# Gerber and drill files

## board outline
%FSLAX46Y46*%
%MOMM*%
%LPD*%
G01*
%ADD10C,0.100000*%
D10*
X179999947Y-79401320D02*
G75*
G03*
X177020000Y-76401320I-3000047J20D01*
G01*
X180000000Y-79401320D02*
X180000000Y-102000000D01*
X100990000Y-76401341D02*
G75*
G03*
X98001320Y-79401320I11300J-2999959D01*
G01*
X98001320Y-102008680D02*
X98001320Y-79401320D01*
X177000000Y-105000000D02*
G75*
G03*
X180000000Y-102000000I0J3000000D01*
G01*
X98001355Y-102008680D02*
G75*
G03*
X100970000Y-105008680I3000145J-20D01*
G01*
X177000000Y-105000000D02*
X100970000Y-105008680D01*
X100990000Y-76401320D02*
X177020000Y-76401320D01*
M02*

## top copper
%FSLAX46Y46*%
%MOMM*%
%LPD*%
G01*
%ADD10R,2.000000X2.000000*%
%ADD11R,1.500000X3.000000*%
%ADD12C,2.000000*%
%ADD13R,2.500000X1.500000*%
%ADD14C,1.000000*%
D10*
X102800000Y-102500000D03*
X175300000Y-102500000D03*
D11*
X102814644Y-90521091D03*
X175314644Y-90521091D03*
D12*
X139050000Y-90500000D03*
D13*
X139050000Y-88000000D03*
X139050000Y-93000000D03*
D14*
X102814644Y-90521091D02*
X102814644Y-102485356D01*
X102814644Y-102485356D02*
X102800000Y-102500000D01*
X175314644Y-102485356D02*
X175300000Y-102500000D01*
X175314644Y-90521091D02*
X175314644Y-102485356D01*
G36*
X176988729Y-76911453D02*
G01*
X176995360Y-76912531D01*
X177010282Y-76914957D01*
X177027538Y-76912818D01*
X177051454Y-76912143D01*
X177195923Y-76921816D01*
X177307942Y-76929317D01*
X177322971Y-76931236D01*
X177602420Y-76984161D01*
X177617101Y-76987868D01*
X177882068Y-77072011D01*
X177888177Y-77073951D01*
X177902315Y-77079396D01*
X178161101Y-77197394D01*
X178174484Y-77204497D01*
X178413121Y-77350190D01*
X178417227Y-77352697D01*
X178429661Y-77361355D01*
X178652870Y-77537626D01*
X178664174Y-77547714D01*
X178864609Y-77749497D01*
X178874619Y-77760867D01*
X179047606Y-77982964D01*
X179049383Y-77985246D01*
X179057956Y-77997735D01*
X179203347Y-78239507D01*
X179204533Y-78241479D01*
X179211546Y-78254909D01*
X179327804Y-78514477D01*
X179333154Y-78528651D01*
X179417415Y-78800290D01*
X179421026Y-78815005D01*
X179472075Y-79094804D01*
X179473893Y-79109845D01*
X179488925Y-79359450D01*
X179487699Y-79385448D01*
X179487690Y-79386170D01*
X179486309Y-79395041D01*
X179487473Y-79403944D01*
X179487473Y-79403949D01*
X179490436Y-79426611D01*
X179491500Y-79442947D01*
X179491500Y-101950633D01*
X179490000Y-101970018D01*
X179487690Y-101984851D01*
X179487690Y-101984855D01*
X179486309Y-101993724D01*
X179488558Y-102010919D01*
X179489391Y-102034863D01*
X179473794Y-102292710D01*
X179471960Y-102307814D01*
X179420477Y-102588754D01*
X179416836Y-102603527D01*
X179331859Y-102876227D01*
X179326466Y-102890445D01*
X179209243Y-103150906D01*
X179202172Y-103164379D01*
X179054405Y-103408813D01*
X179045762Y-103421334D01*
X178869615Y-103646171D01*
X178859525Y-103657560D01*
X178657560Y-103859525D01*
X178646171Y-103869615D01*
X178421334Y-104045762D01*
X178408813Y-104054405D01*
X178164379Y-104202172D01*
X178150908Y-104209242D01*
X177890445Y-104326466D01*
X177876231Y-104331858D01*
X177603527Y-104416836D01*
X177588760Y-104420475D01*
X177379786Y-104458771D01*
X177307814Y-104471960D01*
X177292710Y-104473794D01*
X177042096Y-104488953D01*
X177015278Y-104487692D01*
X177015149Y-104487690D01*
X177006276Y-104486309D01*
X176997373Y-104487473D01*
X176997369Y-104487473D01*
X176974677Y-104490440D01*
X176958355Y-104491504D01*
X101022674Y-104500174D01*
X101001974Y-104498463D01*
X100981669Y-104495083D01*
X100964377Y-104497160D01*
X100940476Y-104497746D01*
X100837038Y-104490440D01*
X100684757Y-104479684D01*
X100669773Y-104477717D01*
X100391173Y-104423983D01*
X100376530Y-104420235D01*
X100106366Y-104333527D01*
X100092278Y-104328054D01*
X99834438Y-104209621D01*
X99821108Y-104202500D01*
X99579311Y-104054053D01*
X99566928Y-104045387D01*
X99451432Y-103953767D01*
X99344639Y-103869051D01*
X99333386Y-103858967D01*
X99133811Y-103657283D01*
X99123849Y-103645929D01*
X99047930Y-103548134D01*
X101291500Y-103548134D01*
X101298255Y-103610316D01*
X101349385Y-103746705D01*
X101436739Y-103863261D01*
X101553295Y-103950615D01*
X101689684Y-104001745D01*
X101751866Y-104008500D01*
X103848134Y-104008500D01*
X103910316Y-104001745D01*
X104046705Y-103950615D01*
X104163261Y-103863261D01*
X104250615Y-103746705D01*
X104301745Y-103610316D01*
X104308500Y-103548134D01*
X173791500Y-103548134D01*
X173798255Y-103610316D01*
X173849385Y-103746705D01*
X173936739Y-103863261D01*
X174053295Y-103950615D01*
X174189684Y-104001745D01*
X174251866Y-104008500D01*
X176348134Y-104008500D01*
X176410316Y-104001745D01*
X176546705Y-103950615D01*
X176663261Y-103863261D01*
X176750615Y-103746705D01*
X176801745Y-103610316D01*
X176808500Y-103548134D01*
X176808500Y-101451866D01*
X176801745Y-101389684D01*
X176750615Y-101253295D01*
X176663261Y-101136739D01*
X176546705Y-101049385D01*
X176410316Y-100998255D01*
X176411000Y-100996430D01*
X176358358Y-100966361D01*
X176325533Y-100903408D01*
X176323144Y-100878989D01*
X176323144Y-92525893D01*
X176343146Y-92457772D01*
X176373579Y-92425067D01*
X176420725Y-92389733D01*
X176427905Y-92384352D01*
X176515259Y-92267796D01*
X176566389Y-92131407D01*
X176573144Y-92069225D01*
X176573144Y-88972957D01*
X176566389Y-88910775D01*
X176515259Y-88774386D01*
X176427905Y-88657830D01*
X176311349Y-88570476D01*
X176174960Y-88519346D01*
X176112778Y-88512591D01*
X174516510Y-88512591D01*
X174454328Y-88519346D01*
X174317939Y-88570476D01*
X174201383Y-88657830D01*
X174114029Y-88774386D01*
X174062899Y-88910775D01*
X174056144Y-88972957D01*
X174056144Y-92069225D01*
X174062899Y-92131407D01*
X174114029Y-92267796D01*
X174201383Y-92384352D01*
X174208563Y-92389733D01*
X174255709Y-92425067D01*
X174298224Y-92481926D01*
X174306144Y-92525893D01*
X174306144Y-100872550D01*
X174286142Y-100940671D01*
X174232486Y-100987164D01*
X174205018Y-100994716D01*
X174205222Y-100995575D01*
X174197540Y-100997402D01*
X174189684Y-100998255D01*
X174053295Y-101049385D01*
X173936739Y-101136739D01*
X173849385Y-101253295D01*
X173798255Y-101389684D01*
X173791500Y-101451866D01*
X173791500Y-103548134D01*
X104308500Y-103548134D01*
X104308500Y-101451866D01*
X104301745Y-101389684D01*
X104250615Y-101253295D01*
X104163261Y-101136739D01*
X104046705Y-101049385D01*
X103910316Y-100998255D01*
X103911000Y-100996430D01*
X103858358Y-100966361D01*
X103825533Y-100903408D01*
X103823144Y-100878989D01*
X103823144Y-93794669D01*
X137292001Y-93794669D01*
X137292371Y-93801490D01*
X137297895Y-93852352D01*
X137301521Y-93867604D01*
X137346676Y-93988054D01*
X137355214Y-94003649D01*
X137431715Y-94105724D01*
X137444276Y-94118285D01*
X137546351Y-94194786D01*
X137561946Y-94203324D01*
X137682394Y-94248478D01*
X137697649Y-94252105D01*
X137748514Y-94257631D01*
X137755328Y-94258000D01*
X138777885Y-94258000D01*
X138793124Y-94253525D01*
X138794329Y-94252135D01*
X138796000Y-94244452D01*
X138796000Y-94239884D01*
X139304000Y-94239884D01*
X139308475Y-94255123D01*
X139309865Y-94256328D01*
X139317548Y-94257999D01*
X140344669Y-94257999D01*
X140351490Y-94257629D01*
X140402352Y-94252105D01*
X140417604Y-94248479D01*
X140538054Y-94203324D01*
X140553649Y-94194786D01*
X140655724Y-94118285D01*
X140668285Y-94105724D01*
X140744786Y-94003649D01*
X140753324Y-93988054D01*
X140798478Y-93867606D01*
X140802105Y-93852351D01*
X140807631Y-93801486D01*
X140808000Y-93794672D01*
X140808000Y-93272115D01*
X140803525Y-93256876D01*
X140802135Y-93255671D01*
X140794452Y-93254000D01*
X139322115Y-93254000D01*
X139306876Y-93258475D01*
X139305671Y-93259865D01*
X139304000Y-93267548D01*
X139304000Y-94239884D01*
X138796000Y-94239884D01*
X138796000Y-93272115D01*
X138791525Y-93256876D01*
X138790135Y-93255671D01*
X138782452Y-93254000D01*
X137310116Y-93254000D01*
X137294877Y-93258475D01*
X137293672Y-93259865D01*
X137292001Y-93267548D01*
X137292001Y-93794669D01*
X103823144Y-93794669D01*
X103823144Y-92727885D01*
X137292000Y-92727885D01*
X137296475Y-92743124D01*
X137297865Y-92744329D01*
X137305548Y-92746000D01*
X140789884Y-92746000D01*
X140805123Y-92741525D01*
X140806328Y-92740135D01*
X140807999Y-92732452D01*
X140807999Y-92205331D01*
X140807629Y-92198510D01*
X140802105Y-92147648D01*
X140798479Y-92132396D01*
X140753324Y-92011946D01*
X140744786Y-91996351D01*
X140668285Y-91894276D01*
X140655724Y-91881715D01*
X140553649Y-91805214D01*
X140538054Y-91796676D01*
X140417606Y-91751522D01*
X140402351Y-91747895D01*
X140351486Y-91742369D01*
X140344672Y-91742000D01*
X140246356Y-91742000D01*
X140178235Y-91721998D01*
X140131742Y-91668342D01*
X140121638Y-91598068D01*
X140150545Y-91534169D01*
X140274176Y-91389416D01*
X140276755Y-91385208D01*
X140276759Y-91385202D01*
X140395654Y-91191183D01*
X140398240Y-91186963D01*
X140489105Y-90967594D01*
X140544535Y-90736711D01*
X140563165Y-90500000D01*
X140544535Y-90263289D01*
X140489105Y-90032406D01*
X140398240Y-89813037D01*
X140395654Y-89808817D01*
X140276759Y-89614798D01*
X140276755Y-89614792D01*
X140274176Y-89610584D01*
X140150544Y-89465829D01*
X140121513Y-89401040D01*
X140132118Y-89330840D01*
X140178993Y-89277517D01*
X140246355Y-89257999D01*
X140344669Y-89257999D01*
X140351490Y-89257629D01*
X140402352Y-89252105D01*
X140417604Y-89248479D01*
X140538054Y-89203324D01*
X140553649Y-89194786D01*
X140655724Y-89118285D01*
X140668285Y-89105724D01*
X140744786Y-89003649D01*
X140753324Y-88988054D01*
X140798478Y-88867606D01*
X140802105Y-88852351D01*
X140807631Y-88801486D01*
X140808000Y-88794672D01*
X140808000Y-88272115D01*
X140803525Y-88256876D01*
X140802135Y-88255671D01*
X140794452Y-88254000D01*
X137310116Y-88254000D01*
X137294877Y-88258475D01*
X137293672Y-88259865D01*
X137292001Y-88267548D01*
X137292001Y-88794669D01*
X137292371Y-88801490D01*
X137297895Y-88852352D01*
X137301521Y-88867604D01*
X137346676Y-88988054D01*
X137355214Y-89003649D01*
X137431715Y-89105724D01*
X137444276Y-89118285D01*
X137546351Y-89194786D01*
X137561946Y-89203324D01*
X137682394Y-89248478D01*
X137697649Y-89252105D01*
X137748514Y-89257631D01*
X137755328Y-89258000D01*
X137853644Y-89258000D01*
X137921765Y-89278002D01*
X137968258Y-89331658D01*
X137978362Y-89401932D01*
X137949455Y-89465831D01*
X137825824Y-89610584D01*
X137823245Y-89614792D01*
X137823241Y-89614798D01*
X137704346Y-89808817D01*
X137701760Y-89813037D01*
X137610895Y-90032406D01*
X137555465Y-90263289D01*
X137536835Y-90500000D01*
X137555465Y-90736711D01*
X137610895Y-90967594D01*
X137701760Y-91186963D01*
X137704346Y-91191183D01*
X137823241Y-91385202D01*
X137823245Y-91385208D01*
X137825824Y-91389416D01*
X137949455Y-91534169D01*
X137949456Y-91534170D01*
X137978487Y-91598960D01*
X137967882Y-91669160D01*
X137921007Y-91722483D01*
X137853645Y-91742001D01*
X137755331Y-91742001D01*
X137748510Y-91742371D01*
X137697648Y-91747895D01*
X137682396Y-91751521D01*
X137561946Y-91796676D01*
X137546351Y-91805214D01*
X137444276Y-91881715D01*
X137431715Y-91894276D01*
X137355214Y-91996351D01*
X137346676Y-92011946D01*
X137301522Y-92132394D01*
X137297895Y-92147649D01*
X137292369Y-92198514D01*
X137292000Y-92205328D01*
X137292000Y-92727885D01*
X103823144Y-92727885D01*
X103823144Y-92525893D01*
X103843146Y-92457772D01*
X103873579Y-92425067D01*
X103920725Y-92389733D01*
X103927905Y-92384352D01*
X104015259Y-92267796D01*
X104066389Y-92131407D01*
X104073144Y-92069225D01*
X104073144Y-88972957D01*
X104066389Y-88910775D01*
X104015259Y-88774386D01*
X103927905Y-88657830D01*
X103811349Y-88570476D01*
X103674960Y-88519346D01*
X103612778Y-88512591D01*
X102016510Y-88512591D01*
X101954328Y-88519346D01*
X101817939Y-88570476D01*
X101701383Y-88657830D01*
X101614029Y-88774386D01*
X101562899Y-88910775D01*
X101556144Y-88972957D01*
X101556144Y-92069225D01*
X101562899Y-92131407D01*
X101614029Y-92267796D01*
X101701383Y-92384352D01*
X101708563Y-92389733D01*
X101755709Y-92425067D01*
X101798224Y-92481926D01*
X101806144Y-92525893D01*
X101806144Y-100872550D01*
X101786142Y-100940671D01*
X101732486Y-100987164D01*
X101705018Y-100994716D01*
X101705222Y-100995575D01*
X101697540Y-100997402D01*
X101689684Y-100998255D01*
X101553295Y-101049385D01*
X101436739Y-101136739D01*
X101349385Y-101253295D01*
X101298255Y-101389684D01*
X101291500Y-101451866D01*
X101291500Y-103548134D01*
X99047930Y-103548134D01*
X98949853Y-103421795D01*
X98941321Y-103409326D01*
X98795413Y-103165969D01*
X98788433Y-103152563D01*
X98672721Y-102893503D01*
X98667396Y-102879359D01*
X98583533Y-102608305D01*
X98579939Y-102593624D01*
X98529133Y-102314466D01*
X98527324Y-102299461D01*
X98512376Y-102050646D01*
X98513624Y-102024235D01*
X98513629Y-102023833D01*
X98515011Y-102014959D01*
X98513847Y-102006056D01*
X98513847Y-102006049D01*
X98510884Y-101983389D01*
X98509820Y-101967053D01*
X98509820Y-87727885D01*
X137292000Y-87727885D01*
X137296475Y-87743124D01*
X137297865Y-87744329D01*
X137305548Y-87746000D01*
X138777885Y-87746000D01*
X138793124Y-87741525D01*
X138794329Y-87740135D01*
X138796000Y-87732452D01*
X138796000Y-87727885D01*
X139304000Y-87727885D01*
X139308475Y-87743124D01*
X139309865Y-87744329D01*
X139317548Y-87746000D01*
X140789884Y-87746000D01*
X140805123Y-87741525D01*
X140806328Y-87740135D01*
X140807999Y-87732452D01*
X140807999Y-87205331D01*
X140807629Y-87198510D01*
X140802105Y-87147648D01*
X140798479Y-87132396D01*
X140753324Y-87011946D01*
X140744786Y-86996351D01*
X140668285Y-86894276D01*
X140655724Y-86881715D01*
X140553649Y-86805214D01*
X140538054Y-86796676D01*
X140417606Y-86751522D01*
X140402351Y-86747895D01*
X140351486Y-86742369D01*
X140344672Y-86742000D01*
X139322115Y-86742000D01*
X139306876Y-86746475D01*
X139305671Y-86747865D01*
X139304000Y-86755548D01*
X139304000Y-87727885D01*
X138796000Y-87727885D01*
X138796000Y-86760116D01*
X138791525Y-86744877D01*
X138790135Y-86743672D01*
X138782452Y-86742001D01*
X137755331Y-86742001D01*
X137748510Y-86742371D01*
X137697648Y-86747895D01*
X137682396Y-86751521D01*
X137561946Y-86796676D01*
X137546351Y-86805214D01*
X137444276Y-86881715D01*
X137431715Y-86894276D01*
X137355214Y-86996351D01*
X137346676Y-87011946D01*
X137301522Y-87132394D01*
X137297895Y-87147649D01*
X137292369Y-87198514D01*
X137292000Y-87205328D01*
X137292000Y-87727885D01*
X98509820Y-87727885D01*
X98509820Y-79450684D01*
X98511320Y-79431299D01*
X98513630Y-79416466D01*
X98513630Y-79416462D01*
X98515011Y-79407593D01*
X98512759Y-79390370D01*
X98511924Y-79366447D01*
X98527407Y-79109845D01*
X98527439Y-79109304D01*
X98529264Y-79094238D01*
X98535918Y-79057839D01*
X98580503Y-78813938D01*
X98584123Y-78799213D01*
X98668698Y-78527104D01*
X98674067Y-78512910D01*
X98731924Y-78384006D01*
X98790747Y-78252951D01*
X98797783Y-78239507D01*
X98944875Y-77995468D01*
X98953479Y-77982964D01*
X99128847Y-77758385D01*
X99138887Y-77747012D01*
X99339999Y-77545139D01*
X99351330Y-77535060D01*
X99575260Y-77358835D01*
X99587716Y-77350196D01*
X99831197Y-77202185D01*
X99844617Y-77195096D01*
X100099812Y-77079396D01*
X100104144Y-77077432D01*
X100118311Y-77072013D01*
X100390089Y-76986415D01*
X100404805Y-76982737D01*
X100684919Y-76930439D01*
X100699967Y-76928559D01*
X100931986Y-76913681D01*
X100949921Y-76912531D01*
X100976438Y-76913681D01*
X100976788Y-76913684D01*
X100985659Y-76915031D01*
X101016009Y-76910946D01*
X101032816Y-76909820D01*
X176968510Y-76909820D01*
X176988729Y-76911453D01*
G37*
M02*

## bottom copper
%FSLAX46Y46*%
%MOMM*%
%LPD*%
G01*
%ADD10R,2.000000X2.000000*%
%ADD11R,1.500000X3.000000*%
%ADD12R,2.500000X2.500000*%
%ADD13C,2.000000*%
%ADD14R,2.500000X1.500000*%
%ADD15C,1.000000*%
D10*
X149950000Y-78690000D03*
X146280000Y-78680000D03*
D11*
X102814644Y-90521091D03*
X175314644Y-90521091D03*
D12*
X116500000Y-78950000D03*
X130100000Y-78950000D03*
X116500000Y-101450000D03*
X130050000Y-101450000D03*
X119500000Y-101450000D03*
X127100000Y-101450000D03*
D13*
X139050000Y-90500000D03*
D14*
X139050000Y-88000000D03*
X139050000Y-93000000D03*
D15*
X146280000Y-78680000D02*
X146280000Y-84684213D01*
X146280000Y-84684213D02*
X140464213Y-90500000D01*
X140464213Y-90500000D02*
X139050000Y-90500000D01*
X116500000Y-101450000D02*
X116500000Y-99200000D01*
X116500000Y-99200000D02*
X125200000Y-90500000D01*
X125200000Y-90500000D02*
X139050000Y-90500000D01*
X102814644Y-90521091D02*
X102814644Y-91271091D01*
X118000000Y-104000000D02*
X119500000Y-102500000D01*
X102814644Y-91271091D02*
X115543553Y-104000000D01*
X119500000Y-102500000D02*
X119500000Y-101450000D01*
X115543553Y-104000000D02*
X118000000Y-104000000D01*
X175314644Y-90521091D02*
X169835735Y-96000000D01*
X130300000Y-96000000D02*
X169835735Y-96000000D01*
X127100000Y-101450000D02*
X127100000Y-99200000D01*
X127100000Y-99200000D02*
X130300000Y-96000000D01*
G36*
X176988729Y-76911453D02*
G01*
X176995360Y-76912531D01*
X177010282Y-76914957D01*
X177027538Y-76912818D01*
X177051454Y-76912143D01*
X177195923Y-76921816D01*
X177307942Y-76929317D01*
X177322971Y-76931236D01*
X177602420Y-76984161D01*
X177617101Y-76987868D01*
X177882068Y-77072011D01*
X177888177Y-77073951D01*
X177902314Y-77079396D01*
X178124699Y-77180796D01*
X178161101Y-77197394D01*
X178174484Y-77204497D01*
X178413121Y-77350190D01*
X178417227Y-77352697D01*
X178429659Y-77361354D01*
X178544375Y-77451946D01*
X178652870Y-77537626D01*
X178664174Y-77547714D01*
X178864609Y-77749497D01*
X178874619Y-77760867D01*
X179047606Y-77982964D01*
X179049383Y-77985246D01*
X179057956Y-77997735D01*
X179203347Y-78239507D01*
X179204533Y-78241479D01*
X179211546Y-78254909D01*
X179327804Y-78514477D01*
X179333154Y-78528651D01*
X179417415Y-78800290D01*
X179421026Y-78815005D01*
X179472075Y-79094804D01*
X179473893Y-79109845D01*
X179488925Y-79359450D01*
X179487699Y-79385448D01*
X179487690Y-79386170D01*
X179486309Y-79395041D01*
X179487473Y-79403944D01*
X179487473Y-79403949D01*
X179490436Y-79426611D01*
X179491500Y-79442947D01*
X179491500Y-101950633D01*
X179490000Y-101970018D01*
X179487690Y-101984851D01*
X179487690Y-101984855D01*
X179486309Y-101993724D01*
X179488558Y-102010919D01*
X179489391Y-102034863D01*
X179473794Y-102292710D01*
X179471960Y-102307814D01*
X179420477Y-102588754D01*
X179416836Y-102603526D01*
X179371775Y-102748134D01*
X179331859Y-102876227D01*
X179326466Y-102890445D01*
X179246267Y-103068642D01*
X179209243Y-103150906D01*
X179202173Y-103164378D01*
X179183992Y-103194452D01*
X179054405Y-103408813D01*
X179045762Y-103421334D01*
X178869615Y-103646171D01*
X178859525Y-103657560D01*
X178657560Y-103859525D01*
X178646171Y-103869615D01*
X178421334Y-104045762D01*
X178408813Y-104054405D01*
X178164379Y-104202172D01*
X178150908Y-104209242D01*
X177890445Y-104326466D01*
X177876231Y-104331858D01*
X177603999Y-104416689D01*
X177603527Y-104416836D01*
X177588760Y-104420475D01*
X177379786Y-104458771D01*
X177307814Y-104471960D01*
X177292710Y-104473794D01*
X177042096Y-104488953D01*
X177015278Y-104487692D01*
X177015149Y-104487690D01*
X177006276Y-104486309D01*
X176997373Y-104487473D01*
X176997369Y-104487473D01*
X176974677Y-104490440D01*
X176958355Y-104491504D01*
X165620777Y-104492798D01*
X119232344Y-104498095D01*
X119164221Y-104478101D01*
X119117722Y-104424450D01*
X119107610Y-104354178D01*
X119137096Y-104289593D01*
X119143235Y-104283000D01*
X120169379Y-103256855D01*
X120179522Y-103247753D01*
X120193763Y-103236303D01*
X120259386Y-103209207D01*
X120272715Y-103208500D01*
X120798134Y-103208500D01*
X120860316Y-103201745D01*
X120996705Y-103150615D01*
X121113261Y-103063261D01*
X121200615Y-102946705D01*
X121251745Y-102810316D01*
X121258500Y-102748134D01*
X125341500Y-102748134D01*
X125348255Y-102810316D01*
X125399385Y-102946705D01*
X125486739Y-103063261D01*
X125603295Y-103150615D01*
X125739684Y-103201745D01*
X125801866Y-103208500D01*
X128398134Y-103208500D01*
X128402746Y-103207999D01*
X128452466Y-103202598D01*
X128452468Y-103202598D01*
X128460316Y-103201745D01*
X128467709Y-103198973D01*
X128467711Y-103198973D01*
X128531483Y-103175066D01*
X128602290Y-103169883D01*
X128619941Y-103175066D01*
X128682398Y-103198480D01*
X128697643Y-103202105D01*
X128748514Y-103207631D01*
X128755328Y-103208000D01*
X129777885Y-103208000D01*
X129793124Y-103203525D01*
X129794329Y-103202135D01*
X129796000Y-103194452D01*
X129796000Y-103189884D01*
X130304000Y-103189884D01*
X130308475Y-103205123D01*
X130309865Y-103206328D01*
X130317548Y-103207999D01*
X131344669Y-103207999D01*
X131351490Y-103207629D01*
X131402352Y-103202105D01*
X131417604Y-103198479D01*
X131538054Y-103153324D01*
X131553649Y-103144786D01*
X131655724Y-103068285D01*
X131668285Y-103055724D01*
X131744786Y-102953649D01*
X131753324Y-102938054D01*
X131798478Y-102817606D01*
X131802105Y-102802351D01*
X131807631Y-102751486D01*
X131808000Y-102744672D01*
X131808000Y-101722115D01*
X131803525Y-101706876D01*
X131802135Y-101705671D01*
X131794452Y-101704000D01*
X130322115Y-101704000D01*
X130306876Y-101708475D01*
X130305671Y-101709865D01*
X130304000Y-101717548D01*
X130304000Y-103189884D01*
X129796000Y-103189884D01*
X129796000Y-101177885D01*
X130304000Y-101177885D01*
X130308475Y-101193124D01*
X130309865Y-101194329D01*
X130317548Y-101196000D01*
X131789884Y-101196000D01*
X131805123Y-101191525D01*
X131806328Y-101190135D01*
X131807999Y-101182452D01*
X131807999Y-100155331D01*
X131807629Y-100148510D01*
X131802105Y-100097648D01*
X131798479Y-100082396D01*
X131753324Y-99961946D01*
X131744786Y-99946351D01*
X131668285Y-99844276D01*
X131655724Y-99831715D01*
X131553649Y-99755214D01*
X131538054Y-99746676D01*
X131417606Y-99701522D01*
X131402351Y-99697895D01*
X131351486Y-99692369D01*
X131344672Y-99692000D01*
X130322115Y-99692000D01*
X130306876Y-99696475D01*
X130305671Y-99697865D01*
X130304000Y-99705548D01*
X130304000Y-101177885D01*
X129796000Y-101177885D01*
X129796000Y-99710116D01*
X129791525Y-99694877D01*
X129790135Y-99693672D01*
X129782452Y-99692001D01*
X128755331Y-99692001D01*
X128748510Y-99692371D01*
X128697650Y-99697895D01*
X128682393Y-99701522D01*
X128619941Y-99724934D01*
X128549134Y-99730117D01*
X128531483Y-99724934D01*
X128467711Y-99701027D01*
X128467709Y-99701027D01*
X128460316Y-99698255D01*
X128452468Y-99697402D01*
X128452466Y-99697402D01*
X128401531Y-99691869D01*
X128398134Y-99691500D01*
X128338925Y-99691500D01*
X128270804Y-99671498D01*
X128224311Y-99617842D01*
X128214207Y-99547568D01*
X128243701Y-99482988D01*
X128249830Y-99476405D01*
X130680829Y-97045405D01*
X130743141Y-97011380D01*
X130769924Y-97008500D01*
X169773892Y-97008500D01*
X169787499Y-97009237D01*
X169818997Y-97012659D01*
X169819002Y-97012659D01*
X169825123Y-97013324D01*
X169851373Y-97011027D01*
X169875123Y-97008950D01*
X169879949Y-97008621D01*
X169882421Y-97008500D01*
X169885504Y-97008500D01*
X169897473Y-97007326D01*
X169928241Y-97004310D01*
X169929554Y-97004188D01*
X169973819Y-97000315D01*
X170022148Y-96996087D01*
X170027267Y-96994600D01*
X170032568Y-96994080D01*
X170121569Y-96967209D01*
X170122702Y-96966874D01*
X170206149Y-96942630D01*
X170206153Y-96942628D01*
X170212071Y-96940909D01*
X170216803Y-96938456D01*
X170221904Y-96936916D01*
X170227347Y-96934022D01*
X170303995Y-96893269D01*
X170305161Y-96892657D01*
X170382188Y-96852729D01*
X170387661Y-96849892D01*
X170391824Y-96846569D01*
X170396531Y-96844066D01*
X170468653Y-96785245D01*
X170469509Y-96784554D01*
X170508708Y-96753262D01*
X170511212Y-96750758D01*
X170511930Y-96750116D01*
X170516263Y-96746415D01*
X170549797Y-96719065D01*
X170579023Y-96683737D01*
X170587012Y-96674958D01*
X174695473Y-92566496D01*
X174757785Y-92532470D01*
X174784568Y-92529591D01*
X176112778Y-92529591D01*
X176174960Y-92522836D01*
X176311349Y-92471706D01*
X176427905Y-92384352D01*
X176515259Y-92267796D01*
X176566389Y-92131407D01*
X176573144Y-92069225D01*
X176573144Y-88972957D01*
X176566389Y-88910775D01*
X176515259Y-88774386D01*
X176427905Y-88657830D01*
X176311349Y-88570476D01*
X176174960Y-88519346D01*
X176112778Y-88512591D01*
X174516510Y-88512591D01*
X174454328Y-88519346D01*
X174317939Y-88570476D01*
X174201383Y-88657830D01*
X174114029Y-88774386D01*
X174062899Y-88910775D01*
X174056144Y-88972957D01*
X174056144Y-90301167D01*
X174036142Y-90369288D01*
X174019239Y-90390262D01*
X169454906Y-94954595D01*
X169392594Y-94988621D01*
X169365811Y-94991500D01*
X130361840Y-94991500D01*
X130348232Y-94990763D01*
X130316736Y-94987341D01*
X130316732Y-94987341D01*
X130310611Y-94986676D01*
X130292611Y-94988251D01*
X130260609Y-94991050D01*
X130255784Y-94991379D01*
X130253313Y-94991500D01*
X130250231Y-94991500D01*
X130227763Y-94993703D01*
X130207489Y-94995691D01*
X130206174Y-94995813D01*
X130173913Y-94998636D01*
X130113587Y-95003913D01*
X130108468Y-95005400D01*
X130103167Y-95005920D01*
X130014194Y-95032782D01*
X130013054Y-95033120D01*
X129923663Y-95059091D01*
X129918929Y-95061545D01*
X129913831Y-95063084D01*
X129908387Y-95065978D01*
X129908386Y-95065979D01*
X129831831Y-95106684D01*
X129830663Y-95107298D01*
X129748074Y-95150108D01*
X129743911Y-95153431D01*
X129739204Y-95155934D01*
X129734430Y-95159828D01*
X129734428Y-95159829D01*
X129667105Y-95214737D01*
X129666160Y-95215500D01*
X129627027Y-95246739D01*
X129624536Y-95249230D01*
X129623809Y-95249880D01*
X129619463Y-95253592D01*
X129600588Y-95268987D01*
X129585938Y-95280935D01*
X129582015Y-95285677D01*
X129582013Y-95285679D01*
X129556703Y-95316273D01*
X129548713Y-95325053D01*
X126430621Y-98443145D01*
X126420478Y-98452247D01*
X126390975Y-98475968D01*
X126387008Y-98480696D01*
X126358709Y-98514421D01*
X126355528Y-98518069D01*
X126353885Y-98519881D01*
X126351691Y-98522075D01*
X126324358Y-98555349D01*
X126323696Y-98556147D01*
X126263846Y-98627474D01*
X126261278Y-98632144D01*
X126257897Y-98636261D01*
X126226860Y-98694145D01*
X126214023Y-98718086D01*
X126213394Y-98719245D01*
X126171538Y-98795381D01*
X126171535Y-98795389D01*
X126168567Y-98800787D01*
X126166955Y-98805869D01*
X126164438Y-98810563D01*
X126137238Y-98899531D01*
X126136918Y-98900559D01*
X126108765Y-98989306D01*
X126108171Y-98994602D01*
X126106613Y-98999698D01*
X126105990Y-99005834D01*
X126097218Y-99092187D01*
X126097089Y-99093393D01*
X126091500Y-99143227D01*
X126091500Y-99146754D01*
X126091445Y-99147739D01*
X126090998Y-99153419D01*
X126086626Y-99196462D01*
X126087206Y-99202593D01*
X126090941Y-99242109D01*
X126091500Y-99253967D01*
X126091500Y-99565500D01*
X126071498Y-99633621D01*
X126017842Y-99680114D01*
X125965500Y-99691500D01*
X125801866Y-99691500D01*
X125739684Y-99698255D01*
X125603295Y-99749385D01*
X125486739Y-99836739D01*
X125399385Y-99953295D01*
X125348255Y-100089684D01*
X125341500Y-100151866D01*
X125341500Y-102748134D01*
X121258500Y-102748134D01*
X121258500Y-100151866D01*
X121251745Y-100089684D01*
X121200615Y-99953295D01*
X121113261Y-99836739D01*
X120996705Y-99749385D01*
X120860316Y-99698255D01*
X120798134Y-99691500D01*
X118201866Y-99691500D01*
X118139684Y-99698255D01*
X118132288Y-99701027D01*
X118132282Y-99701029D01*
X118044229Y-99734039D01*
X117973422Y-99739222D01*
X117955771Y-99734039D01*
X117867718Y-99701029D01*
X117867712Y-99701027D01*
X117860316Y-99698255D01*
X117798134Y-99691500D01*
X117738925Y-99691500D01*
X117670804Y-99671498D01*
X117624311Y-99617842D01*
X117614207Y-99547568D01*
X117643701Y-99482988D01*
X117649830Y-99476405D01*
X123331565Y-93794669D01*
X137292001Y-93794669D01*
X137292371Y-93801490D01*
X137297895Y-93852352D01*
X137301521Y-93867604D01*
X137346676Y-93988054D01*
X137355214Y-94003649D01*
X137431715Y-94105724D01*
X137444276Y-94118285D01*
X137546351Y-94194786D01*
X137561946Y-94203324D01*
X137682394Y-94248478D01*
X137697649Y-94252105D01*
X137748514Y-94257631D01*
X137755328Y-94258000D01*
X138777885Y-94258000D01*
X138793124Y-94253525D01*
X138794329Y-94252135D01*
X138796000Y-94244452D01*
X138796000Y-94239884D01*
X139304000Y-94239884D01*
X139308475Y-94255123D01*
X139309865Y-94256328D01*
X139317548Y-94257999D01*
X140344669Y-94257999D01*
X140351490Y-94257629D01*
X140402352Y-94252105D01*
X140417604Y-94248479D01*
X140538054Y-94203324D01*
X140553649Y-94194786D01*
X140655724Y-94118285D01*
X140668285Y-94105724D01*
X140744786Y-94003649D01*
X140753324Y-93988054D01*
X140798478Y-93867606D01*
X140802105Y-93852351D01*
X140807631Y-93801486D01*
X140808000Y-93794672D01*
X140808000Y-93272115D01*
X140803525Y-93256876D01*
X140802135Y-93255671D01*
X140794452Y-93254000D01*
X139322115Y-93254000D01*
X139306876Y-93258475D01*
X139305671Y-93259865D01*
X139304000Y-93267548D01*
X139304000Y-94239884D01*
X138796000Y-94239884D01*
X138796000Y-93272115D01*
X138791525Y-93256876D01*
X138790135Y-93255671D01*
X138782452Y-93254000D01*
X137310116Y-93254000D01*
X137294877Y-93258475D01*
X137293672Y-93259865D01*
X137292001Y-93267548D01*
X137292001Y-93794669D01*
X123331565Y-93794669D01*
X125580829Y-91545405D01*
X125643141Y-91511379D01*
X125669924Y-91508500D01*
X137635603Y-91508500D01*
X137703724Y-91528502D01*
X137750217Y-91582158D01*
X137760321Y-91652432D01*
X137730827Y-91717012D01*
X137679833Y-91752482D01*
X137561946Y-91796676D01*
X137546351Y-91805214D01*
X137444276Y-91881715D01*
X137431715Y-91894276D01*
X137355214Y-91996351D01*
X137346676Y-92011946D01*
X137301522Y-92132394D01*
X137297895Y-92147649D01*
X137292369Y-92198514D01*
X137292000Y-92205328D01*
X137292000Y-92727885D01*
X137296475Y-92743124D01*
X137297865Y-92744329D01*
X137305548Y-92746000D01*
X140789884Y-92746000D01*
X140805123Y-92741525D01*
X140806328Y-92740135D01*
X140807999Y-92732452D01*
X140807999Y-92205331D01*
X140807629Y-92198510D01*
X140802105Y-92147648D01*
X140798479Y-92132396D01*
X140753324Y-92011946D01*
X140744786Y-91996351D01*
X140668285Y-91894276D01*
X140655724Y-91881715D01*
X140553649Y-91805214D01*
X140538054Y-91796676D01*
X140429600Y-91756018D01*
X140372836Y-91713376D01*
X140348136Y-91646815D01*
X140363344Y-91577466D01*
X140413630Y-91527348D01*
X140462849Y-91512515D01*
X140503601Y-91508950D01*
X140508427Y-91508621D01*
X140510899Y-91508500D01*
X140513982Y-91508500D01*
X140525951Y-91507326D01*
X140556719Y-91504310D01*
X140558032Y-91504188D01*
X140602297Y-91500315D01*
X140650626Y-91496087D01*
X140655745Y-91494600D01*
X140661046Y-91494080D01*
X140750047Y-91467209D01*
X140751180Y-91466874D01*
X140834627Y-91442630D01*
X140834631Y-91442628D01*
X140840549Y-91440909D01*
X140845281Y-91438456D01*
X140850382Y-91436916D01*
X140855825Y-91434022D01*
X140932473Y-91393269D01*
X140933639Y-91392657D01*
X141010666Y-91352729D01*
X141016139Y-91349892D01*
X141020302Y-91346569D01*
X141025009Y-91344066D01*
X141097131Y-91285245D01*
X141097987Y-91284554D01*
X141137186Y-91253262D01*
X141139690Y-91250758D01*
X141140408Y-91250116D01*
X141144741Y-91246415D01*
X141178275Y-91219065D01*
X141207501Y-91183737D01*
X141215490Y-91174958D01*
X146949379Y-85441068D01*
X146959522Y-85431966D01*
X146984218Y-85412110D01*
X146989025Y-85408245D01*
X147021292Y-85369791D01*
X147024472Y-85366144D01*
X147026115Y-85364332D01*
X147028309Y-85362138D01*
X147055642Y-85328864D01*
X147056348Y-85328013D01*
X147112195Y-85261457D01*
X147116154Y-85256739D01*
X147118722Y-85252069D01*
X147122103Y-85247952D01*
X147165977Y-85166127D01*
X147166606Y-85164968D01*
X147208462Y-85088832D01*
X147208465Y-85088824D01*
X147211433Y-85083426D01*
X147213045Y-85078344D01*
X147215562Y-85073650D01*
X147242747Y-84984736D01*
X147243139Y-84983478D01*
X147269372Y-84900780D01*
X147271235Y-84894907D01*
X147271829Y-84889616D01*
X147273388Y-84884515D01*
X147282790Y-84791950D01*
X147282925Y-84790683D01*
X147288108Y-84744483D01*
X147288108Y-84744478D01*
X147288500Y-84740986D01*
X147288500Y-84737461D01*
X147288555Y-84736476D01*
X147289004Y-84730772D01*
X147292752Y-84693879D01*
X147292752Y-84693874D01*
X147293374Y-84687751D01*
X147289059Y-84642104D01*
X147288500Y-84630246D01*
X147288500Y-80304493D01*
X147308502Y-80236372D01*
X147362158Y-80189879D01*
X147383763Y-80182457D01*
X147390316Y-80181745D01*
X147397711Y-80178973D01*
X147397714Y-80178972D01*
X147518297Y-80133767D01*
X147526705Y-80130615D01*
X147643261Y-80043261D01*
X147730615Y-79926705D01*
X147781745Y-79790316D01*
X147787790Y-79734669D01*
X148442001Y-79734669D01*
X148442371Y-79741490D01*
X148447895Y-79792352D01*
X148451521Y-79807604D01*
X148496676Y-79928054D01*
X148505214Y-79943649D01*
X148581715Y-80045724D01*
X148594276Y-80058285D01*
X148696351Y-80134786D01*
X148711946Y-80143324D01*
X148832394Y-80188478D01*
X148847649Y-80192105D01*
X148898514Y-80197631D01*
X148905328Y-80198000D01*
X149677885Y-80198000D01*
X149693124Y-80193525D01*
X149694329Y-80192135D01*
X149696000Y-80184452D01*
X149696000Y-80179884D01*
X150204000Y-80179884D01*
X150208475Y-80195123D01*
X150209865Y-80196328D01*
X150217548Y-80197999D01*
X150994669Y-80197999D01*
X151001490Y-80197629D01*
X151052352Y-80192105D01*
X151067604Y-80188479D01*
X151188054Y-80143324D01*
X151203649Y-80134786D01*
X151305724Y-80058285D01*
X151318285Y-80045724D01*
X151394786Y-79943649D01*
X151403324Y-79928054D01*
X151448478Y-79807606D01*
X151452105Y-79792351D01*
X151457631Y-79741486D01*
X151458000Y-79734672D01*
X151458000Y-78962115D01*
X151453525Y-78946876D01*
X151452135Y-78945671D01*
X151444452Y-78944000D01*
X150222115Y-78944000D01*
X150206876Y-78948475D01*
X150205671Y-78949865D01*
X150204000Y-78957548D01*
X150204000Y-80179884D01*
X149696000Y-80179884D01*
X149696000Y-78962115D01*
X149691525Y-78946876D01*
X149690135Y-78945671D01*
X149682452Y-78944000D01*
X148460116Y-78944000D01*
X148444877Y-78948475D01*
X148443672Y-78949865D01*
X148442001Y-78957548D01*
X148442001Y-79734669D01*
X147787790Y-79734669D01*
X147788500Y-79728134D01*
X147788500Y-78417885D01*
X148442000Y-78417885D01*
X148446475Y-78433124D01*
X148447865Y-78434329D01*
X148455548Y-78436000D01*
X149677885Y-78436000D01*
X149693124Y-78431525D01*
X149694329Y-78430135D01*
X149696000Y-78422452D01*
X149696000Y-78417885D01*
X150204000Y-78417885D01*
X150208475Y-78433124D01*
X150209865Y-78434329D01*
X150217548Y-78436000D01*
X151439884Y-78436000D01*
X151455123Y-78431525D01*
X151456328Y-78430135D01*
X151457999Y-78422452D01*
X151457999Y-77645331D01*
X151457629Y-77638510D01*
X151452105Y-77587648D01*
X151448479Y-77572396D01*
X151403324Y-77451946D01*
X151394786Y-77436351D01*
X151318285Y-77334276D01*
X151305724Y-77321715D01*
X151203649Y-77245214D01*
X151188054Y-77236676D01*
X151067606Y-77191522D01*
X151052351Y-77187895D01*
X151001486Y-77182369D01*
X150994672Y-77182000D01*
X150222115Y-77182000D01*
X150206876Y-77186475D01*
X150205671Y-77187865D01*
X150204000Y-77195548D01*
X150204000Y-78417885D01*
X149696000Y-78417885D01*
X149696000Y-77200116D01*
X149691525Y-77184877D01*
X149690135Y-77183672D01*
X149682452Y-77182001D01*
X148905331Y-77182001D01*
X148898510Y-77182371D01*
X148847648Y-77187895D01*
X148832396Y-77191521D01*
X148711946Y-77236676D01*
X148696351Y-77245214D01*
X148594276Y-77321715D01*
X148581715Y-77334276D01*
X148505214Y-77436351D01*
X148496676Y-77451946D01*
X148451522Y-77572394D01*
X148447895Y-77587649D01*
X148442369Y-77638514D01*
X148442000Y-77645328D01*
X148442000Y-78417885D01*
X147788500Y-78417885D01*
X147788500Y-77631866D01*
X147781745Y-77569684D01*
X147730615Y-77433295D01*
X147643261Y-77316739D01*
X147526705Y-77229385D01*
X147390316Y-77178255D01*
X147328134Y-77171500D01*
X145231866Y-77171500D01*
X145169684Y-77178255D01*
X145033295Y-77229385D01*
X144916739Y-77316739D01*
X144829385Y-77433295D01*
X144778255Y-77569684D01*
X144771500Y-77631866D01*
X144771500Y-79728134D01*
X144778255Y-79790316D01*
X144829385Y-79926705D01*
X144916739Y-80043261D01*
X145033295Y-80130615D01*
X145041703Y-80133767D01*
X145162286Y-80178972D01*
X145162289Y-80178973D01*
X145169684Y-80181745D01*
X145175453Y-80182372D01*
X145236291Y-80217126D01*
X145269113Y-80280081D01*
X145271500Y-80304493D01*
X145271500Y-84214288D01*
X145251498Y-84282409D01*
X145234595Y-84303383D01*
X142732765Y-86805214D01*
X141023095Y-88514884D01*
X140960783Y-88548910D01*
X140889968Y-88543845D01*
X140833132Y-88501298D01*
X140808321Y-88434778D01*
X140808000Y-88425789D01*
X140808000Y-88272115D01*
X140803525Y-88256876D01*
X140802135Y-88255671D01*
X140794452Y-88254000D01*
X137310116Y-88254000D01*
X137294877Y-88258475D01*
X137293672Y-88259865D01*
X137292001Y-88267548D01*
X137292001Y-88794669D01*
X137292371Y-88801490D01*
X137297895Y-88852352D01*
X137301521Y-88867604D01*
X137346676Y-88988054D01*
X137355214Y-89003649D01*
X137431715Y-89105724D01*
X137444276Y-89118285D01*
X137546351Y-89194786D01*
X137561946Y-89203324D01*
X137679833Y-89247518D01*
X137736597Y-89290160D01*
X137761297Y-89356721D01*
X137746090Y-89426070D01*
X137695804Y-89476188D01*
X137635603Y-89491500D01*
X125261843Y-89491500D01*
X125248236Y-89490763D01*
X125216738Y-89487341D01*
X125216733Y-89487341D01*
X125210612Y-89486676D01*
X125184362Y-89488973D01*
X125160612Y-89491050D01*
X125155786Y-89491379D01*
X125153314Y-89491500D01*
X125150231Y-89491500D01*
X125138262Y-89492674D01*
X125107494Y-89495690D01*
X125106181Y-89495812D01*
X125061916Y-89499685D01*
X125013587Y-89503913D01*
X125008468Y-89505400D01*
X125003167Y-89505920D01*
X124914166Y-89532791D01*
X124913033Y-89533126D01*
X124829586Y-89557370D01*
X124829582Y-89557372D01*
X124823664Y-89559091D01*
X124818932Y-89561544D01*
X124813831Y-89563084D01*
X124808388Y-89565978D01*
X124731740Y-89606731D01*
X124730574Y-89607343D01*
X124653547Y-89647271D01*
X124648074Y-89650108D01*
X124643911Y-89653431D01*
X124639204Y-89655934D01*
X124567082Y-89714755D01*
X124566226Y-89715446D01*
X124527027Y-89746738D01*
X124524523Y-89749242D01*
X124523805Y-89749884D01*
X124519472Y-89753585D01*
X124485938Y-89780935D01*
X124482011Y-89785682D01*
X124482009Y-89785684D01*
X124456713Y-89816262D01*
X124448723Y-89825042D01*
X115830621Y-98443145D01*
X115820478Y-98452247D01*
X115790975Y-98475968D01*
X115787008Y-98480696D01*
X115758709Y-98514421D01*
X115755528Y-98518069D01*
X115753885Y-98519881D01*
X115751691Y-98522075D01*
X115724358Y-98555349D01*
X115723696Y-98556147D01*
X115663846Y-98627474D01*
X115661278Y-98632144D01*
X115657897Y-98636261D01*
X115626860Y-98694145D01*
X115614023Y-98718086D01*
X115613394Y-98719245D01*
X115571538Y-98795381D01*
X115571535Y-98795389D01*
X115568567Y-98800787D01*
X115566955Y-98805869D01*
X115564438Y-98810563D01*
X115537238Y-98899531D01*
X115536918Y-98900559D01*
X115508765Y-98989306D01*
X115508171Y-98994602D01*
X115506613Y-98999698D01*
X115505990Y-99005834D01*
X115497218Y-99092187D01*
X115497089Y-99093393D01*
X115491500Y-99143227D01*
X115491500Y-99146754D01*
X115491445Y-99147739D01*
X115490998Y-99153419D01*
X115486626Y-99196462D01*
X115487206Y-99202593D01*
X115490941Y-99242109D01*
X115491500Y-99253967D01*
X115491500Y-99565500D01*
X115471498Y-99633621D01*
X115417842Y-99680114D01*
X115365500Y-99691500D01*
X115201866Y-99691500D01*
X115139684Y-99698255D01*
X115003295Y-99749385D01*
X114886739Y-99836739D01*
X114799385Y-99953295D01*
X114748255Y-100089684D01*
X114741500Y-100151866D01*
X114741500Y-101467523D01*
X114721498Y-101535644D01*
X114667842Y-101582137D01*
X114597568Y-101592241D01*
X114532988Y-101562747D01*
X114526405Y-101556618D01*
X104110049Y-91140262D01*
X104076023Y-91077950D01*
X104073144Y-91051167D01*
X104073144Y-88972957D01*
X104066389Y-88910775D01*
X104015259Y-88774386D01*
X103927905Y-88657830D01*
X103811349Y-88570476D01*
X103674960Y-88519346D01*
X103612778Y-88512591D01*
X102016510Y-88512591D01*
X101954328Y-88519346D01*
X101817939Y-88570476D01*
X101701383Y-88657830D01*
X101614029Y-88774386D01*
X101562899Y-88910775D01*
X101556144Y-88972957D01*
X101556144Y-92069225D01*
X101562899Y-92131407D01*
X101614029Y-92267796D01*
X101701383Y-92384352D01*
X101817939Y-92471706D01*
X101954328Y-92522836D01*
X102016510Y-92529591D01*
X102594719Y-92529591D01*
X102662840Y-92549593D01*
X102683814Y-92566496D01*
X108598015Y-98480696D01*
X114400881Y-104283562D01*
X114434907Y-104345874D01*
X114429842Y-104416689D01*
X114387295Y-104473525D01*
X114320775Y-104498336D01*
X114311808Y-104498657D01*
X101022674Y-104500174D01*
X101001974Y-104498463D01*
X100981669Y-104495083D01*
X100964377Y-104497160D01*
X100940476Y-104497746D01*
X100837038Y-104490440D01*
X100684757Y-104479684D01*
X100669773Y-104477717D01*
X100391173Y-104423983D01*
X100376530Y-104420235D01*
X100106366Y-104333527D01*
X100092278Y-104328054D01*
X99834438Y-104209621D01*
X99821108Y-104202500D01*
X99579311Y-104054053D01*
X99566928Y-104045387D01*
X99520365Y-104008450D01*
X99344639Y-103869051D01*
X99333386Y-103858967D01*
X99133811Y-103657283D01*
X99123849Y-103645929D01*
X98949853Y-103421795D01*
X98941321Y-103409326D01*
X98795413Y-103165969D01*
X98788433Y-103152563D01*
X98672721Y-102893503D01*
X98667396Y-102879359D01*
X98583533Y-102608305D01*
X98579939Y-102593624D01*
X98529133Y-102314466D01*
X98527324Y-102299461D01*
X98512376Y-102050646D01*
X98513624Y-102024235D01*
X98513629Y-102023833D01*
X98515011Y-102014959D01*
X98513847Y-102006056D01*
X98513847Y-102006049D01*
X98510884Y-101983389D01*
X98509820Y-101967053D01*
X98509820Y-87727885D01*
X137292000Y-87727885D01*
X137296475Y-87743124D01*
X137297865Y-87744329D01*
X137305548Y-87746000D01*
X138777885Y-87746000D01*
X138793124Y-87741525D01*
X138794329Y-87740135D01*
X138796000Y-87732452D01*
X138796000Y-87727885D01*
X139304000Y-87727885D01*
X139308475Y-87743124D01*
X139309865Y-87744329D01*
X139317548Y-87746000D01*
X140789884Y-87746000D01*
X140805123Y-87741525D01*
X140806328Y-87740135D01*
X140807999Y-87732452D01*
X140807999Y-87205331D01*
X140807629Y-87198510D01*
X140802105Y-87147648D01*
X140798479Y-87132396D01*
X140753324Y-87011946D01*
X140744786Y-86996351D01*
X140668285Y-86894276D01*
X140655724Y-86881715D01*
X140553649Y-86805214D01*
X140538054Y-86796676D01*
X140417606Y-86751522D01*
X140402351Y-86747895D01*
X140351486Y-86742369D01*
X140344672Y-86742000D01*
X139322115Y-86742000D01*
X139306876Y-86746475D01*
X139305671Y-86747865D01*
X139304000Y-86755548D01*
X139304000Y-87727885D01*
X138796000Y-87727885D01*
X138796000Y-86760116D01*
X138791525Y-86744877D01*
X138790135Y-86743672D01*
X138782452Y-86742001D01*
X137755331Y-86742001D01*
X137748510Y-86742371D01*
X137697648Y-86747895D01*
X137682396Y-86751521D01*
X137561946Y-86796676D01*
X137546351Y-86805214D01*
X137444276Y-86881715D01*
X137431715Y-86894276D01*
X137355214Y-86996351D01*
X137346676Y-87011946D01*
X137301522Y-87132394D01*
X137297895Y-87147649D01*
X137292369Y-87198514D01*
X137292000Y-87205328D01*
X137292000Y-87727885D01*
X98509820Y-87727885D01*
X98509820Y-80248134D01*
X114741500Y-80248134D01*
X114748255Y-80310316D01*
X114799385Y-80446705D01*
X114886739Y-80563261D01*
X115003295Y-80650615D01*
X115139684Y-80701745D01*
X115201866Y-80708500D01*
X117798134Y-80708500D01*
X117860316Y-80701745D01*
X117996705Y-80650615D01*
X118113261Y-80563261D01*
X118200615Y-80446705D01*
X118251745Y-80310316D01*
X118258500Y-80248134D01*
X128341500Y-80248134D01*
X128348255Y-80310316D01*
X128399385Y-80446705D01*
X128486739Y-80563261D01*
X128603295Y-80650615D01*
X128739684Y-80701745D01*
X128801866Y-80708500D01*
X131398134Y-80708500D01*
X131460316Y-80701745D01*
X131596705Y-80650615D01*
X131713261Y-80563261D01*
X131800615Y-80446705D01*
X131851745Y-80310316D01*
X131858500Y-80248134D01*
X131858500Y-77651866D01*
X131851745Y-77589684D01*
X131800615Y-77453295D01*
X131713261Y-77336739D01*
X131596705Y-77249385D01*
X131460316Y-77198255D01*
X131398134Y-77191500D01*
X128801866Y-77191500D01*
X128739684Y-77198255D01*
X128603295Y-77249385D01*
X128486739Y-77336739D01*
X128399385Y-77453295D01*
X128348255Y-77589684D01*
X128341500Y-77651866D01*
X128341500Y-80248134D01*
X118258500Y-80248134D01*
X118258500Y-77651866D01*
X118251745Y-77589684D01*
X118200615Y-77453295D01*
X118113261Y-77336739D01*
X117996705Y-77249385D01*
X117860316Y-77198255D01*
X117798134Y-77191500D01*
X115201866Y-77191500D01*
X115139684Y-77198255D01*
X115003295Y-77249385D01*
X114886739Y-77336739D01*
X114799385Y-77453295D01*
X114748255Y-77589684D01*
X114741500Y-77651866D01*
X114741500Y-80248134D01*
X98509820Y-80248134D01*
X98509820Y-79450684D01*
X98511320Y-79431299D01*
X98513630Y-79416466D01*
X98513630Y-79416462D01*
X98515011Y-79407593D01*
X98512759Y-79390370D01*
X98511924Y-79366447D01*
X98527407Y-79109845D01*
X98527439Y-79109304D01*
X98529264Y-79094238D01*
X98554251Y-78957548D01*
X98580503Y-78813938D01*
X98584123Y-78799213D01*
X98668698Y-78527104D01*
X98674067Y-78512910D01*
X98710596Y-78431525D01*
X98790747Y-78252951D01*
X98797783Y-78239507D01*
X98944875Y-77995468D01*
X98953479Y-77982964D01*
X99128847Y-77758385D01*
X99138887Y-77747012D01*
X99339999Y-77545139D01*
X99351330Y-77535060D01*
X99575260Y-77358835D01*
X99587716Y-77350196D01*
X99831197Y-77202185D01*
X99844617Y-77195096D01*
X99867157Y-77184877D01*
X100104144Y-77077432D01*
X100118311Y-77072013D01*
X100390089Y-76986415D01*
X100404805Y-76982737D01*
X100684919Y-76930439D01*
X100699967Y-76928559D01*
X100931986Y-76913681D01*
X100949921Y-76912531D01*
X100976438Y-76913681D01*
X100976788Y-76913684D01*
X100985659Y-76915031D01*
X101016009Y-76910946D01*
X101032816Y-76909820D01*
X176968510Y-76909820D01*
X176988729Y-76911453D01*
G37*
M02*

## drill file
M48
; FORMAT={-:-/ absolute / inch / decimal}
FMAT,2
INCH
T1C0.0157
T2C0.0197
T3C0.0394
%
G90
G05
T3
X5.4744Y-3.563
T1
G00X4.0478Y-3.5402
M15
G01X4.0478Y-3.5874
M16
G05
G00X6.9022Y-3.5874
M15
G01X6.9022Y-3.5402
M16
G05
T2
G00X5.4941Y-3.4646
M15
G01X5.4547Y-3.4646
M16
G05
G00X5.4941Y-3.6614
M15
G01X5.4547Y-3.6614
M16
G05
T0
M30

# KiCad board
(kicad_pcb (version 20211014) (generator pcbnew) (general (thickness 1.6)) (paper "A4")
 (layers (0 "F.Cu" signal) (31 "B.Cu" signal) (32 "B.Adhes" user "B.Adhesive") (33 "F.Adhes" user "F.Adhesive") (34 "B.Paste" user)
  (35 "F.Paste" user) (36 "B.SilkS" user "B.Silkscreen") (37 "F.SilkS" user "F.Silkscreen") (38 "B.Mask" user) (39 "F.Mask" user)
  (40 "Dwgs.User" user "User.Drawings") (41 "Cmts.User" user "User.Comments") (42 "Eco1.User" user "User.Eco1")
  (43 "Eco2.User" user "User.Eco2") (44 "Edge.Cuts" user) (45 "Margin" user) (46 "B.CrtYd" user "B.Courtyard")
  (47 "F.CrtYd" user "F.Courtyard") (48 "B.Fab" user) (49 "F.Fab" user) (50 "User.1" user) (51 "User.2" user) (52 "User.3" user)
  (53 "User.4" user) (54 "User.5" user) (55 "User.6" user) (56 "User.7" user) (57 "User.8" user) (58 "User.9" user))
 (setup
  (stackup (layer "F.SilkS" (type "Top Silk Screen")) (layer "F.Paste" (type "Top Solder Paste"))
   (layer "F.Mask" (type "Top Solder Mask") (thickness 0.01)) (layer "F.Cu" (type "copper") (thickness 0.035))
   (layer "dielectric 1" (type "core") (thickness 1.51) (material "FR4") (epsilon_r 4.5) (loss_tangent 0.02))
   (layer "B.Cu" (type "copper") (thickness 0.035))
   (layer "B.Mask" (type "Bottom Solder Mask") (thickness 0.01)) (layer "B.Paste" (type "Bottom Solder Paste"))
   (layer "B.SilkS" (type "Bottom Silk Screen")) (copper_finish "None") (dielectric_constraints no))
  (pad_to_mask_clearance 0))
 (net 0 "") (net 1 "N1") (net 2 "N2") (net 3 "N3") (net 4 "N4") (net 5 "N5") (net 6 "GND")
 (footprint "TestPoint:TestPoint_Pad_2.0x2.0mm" (layer "F.Cu") (at 102.8 102.5)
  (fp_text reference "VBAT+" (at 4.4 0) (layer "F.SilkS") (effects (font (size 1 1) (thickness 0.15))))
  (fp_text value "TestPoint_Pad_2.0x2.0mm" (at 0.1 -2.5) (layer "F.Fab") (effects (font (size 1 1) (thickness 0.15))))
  (pad "1" smd rect (at 0 0) (size 2 2) (layers "F.Cu" "F.Mask") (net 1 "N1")))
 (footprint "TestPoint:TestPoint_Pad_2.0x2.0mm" (layer "F.Cu") (at 175.3 102.5)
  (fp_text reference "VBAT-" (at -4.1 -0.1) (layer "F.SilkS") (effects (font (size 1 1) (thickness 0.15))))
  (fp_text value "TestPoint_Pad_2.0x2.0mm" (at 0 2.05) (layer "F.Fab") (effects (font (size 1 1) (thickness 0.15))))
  (pad "1" smd rect (at 0 0) (size 2 2) (layers "F.Cu" "F.Mask") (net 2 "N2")))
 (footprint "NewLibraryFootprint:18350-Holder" (layer "F.Cu") (at 175.314644 90.521091)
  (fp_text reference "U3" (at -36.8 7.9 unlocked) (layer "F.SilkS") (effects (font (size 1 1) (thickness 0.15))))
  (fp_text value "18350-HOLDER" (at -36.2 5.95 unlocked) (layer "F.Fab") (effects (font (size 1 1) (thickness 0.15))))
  (pad "1" thru_hole rect (at -72.5 0 270) (size 3 1.5) (drill oval 1.6 0.4) (layers *.Cu *.Mask) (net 1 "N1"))
  (pad "2" thru_hole rect (at 0 0 90) (size 3 1.5) (drill oval 1.6 0.4) (layers *.Cu *.Mask) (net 2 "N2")))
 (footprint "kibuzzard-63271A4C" (layer "F.Cu") (at 123.3 79 180)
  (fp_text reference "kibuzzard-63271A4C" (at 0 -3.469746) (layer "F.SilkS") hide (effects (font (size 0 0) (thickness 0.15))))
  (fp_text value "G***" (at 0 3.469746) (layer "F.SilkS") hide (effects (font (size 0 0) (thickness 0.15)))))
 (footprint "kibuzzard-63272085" (layer "B.Cu") (at 154.35 78.72 180)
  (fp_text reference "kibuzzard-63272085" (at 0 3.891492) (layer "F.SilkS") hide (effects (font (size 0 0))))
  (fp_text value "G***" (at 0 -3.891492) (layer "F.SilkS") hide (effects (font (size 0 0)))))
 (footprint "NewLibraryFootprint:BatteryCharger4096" (layer "B.Cu") (at 123.3 101.45 -90)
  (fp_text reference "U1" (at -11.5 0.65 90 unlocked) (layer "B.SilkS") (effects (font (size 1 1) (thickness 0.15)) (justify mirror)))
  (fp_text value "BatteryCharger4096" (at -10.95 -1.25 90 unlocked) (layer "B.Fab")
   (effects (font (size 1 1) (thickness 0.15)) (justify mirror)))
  (pad "1" smd rect (at -22.5 6.8 270) (size 2.5 2.5) (layers "B.Cu" "B.Paste" "B.Mask") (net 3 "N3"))
  (pad "2" smd rect (at -22.5 -6.8 270) (size 2.5 2.5) (layers "B.Cu" "B.Paste" "B.Mask") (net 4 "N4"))
  (pad "3" smd rect (at 0 6.8 270) (size 2.5 2.5) (layers "B.Cu" "B.Paste" "B.Mask") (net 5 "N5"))
  (pad "4" smd rect (at 0 -6.75 270) (size 2.5 2.5) (layers "B.Cu" "B.Paste" "B.Mask") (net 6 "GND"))
  (pad "5" smd rect (at 0 3.8 270) (size 2.5 2.5) (layers "B.Cu" "B.Paste" "B.Mask") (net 1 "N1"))
  (pad "6" smd rect (at 0 -3.8 270) (size 2.5 2.5) (layers "B.Cu" "B.Paste" "B.Mask") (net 2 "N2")))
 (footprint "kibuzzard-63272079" (layer "B.Cu") (at 141.88 78.72 180)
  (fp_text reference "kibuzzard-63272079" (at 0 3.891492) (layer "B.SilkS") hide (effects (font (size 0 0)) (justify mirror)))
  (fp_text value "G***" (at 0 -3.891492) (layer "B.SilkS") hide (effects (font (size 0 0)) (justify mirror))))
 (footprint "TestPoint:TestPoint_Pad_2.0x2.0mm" (layer "B.Cu") (at 149.95 78.69 180)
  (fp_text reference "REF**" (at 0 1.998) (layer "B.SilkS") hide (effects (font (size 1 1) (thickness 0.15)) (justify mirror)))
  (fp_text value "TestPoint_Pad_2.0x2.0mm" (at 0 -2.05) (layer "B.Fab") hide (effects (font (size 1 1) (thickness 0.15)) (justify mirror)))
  (pad "1" smd rect (at 0 0 180) (size 2 2) (layers "B.Cu" "B.Mask") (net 6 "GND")))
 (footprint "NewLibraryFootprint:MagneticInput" (layer "B.Cu") (at 139.05 90.5 -90)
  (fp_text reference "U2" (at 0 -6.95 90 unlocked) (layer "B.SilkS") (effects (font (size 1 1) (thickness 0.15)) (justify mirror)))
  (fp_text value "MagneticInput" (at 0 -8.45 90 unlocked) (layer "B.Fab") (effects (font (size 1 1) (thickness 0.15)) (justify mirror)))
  (pad "1" thru_hole circle (at 0 0 180) (size 2 2) (drill 1) (layers *.Cu *.Mask) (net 5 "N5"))
  (pad "2" thru_hole rect (at -2.5 0 180) (size 2.5 1.5) (drill oval 1.5 0.5) (layers *.Cu *.Mask) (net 6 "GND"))
  (pad "3" thru_hole rect (at 2.5 0 180) (size 2.5 1.5) (drill oval 1.5 0.5) (layers *.Cu *.Mask) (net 6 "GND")))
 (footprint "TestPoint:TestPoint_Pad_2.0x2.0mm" (layer "B.Cu") (at 146.28 78.68 180)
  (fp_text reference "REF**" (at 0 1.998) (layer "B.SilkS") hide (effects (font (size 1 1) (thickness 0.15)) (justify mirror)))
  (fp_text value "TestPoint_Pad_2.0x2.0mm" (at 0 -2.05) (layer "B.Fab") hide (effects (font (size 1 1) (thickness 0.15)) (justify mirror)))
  (pad "1" smd rect (at 0 0 180) (size 2 2) (layers "B.Cu" "B.Mask") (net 5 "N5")))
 (gr_arc (start 177.02 76.40132) (mid 179.128383 77.287059) (end 180 79.40132) (layer "Edge.Cuts") (width 0.1))
 (gr_line (start 180 79.40132) (end 180 102) (layer "Edge.Cuts") (width 0.1))
 (gr_arc (start 98.00132 79.40132) (mid 98.876 77.283998) (end 100.99 76.40132) (layer "Edge.Cuts") (width 0.1))
 (gr_line (start 98.00132 102.00868) (end 98.00132 79.40132) (layer "Edge.Cuts") (width 0.1))
 (gr_arc (start 180 102) (mid 179.12132 104.12132) (end 177 105) (layer "Edge.Cuts") (width 0.1))
 (gr_arc (start 100.97 105.00868) (mid 98.868938 104.118963) (end 98.00132 102.00868) (layer "Edge.Cuts") (width 0.1))
 (gr_line (start 177 105) (end 100.97 105.00868) (layer "Edge.Cuts") (width 0.1))
 (gr_line (start 100.99 76.40132) (end 177.02 76.40132) (layer "Edge.Cuts") (width 0.1))
 (segment (start 116.5 101.45) (end 116.5 99.2) (width 1) (layer "B.Cu") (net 5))
 (segment (start 146.28 84.684213) (end 140.464213 90.5) (width 1) (layer "B.Cu") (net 5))
 (segment (start 146.28 78.68) (end 146.28 84.684213) (width 1) (layer "B.Cu") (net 5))
 (segment (start 140.464213 90.5) (end 139.05 90.5) (width 1) (layer "B.Cu") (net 5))
 (segment (start 116.5 99.2) (end 125.2 90.5) (width 1) (layer "B.Cu") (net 5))
 (segment (start 125.2 90.5) (end 139.05 90.5) (width 1) (layer "B.Cu") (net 5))
 (segment (start 102.814644 90.521091) (end 102.814644 102.485356) (width 1) (layer "F.Cu") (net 1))
 (segment (start 102.814644 102.485356) (end 102.8 102.5) (width 1) (layer "F.Cu") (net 1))
 (segment (start 102.814644 90.521091) (end 102.814644 91.271091) (width 1) (layer "B.Cu") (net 1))
 (segment (start 118 104) (end 119.5 102.5) (width 1) (layer "B.Cu") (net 1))
 (segment (start 102.814644 91.271091) (end 115.543553 104) (width 1) (layer "B.Cu") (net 1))
 (segment (start 119.5 102.5) (end 119.5 101.45) (width 1) (layer "B.Cu") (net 1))
 (segment (start 115.543553 104) (end 118 104) (width 1) (layer "B.Cu") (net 1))
 (segment (start 175.314644 102.485356) (end 175.3 102.5) (width 1) (layer "F.Cu") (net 2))
 (segment (start 175.314644 90.521091) (end 175.314644 102.485356) (width 1) (layer "F.Cu") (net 2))
 (segment (start 175.314644 90.521091) (end 169.835735 96) (width 1) (layer "B.Cu") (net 2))
 (segment (start 130.3 96) (end 169.835735 96) (width 1) (layer "B.Cu") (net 2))
 (segment (start 127.1 101.45) (end 127.1 99.2) (width 1) (layer "B.Cu") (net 2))
 (segment (start 127.1 99.2) (end 130.3 96) (width 1) (layer "B.Cu") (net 2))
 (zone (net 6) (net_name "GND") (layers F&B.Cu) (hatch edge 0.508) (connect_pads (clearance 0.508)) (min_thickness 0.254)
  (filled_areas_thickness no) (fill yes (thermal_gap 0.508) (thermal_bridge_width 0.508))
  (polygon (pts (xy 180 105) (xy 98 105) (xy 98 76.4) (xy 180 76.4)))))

